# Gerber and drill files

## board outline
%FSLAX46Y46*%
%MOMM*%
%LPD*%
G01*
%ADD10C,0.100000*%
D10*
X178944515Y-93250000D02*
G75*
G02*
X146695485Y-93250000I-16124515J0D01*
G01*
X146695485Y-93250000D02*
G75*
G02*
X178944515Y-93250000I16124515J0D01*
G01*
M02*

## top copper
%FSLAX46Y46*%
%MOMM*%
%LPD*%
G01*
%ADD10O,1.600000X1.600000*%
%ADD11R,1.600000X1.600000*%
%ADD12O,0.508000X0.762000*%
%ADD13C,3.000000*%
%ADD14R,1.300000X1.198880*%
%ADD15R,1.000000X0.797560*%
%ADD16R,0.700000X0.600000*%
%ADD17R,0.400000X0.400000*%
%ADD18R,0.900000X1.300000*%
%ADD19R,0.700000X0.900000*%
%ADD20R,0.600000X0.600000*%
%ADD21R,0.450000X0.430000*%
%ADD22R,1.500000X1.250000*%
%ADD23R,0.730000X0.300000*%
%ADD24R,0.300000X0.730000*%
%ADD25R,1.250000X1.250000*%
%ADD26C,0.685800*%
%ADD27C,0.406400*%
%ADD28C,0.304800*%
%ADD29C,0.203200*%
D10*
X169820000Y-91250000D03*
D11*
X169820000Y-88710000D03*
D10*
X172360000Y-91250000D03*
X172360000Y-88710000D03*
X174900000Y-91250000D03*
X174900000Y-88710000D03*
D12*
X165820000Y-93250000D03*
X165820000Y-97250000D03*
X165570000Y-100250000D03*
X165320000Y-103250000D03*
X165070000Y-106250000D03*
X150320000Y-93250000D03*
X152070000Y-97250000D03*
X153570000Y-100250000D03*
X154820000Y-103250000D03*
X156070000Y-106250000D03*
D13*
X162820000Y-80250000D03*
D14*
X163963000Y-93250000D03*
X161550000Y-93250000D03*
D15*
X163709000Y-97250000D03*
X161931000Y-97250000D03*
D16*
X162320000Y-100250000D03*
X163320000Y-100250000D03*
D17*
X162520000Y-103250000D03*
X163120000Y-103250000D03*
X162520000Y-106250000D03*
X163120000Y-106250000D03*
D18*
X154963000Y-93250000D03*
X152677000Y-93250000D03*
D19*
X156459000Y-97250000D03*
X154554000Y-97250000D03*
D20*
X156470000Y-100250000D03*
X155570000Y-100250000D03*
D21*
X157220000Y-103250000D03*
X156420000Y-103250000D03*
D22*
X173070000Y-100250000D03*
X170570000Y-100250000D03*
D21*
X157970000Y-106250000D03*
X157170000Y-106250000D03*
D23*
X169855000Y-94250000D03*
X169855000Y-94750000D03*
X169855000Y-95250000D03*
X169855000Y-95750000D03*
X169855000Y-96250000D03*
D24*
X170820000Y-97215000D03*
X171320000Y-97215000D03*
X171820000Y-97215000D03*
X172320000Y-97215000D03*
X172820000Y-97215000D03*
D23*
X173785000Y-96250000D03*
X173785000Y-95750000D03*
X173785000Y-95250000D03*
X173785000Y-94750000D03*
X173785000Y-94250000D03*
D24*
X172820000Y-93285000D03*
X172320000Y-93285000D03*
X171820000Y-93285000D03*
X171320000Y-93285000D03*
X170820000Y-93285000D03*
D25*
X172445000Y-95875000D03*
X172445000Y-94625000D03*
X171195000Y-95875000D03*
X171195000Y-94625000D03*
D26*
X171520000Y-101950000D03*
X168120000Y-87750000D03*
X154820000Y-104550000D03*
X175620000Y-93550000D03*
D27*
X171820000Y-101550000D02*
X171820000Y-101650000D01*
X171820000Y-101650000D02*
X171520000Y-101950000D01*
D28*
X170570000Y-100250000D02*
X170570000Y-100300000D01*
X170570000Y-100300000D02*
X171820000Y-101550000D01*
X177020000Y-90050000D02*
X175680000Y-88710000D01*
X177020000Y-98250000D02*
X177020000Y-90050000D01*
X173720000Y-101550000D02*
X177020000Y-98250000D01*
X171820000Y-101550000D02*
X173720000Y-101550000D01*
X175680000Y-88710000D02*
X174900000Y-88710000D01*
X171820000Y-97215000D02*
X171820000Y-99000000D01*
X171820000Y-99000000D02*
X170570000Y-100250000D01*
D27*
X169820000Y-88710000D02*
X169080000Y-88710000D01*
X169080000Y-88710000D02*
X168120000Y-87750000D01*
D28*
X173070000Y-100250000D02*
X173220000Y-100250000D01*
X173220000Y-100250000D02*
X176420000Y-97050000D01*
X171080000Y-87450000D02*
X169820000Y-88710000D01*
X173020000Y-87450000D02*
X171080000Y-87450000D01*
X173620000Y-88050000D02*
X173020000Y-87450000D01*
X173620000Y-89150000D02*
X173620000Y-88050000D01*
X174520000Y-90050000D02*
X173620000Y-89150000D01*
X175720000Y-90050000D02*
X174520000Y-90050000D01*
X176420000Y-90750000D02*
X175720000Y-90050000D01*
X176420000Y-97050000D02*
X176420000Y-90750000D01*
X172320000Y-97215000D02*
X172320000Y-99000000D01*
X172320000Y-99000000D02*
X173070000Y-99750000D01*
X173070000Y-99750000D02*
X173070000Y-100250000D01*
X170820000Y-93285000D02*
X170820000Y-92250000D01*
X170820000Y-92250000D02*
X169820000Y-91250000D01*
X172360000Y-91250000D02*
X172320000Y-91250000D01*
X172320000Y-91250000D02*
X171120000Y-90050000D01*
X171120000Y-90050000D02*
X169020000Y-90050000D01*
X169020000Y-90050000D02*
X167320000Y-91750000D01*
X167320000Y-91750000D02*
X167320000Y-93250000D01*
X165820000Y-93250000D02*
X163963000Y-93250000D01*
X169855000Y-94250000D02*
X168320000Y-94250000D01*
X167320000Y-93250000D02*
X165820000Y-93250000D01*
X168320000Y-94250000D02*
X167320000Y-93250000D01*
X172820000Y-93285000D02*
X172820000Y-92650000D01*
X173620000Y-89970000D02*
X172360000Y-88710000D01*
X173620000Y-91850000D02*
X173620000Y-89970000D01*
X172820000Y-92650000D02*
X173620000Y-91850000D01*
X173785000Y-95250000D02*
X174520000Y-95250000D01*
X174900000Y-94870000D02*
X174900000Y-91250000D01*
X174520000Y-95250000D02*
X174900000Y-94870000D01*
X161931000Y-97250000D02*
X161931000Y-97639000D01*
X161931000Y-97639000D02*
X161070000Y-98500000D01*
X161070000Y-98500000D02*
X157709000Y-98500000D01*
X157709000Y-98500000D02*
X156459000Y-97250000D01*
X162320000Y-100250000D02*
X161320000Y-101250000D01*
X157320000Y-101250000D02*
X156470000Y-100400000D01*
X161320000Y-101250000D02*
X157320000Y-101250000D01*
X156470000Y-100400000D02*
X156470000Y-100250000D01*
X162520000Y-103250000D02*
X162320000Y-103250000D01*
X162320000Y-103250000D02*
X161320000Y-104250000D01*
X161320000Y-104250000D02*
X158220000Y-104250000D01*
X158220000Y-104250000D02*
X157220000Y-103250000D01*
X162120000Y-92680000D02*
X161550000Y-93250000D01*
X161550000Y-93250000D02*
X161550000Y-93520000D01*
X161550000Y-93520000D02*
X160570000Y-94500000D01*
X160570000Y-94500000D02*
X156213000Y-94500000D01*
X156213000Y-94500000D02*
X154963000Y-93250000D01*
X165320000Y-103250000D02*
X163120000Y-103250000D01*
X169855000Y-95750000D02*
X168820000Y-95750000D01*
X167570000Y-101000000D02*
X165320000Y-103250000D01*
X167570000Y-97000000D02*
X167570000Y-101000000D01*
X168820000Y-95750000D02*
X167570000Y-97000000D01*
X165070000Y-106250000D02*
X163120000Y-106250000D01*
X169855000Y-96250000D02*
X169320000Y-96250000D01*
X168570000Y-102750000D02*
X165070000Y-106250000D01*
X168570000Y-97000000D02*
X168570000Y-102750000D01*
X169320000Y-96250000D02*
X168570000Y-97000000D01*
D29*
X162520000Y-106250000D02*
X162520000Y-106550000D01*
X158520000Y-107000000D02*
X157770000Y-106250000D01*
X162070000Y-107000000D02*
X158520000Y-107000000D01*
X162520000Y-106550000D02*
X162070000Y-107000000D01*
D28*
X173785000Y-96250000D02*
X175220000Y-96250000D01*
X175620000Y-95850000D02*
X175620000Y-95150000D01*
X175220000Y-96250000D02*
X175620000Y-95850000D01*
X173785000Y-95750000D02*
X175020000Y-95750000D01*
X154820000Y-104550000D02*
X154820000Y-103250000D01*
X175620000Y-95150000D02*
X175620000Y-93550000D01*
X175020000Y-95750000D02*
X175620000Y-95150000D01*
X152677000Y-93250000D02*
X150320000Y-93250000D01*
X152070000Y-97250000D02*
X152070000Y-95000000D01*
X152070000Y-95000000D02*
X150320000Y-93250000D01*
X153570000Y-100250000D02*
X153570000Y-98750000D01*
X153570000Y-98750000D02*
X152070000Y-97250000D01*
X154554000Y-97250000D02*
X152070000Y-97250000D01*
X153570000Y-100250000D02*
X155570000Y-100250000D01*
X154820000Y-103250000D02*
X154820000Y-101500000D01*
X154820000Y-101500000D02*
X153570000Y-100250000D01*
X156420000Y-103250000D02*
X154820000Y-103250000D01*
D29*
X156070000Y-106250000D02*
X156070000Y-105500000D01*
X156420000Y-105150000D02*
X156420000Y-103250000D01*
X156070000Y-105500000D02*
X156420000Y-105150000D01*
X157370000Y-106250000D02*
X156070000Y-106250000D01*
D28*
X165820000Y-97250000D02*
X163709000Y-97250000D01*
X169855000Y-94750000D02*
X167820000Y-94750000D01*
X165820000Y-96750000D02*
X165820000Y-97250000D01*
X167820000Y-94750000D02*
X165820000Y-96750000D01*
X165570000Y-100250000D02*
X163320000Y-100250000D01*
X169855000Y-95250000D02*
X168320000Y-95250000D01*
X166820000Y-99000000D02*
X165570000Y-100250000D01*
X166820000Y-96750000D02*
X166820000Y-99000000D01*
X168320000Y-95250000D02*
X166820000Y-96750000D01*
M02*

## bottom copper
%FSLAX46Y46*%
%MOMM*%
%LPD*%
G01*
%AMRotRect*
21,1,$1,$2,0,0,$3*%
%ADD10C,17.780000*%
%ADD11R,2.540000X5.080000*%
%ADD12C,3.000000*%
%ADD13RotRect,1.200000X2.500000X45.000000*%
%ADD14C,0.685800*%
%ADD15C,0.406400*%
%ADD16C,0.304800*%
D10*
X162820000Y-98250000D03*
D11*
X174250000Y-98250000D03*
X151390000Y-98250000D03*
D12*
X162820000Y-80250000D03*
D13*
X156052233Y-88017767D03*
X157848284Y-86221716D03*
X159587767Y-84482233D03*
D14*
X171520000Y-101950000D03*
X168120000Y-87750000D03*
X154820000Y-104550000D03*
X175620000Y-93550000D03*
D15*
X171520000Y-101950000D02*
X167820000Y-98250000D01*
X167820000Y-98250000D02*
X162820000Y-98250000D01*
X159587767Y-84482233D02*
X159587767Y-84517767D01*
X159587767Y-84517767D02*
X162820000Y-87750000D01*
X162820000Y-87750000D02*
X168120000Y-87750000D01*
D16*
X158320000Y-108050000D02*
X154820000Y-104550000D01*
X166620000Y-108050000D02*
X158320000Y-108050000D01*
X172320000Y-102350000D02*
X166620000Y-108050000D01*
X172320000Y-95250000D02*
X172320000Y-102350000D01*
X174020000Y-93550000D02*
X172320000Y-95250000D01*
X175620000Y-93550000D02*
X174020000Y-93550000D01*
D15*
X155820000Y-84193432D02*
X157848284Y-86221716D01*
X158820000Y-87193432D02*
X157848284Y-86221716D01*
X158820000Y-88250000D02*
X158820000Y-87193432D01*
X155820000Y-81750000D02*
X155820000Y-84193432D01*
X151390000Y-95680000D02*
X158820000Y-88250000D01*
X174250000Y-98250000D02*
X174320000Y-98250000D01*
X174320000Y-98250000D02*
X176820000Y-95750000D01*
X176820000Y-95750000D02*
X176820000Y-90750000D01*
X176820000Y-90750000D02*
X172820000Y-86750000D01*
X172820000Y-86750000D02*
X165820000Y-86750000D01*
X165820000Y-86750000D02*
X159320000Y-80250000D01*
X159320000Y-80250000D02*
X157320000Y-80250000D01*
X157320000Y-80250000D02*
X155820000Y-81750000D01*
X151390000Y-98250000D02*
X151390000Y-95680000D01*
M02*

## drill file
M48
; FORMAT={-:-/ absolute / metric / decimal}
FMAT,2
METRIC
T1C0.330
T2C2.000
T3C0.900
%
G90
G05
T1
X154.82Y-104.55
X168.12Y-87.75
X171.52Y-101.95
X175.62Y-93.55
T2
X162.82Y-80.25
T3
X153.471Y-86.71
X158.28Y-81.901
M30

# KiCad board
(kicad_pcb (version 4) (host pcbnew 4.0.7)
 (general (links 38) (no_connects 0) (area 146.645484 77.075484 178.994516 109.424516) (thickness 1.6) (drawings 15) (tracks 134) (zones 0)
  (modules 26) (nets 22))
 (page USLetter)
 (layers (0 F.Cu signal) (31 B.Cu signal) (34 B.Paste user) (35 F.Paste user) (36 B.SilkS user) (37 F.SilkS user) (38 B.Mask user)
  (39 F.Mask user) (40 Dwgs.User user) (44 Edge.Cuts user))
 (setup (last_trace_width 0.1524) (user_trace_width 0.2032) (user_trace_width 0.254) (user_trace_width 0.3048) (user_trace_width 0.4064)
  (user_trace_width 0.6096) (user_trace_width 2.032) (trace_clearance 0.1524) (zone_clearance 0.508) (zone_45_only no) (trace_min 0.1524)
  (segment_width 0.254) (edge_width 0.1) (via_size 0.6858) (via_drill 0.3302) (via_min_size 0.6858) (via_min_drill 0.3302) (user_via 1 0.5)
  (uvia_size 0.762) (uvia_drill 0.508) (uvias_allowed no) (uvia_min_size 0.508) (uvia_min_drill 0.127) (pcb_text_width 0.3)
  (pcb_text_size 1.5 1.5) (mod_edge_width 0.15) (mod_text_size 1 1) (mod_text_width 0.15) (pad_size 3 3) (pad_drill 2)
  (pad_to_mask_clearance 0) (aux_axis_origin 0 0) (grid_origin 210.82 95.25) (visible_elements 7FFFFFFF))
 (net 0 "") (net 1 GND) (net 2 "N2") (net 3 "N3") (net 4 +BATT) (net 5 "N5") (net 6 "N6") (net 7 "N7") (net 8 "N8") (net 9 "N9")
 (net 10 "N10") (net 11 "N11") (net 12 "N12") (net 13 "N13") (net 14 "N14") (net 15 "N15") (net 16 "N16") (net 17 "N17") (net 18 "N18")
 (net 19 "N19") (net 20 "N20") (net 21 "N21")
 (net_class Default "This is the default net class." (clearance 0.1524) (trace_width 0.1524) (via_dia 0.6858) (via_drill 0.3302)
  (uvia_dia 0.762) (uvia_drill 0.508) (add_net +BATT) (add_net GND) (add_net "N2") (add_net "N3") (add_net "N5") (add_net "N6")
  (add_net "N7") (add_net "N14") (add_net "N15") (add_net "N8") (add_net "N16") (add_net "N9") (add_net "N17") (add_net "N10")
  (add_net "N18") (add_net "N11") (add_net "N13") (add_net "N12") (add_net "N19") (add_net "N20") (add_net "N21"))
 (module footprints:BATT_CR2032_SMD (layer B.Cu) (at 162.82 98.25 180)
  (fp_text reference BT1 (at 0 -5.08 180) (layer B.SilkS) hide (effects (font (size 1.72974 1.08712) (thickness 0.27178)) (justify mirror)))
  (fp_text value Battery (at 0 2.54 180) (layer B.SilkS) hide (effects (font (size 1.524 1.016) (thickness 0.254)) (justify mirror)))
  (pad 2 smd circle (at 0 0 180) (size 17.78 17.78) (layers B.Cu B.Paste B.Mask) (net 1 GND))
  (pad 1 smd rect (at -11.43 0 180) (size 2.54 5.08) (layers B.Cu B.Paste B.Mask) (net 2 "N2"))
  (pad 1 smd rect (at 11.43 0 180) (size 2.54 5.08) (layers B.Cu B.Paste B.Mask) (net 2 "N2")))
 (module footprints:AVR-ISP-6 (layer F.Cu) (at 169.82 91.25 90)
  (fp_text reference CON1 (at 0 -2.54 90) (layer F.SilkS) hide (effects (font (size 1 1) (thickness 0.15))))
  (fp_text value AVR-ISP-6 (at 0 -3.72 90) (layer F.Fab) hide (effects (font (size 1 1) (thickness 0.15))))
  (pad 1 smd oval (at 0 0 90) (size 1.6 1.6) (layers F.Cu F.Paste F.Mask) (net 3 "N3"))
  (pad 2 smd rect (at 2.54 0 90) (size 1.6 1.6) (layers F.Cu F.Paste F.Mask) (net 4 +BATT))
  (pad 3 smd oval (at 0 2.54 90) (size 1.6 1.6) (layers F.Cu F.Paste F.Mask) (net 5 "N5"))
  (pad 4 smd oval (at 2.54 2.54 90) (size 1.6 1.6) (layers F.Cu F.Paste F.Mask) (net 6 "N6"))
  (pad 5 smd oval (at 0 5.08 90) (size 1.6 1.6) (layers F.Cu F.Paste F.Mask) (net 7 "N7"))
  (pad 6 smd oval (at 2.54 5.08 90) (size 1.6 1.6) (layers F.Cu F.Paste F.Mask) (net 1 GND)))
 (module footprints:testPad (layer F.Cu) (at 165.82 93.25)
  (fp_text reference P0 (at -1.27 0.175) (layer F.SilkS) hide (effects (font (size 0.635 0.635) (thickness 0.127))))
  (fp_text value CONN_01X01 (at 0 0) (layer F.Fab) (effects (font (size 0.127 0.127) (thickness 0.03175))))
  (pad 1 smd oval (at 0 0) (size 0.508 0.762) (layers F.Cu F.Paste F.Mask) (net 5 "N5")))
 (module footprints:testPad (layer F.Cu) (at 165.82 97.25)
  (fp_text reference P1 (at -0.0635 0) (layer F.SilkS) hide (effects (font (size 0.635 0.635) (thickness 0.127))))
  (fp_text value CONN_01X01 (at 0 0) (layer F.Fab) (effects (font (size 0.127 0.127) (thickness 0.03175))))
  (pad 1 smd oval (at 0 0) (size 0.508 0.762) (layers F.Cu F.Paste F.Mask) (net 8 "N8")))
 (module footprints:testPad (layer F.Cu) (at 165.57 100.25)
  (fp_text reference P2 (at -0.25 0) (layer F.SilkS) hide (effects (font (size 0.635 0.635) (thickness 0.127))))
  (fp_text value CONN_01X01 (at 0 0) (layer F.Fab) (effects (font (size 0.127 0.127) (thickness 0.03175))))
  (pad 1 smd oval (at 0 0) (size 0.508 0.762) (layers F.Cu F.Paste F.Mask) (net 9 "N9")))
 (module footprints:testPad (layer F.Cu) (at 165.32 103.25)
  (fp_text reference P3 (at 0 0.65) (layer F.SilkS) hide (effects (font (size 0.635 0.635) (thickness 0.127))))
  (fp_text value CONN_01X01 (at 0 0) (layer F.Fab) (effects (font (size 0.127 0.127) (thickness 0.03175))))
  (pad 1 smd oval (at 0 0) (size 0.508 0.762) (layers F.Cu F.Paste F.Mask) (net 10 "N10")))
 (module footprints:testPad (layer F.Cu) (at 165.07 106.25)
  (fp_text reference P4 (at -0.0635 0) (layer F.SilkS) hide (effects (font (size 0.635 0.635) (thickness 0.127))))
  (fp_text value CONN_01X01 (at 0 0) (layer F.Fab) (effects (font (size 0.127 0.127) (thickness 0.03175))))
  (pad 1 smd oval (at 0 0) (size 0.508 0.762) (layers F.Cu F.Paste F.Mask) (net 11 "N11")))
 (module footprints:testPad (layer F.Cu) (at 150.32 93.25)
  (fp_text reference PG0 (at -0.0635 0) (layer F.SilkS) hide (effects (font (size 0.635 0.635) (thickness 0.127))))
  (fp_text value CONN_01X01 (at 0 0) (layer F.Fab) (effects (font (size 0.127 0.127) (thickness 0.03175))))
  (pad 1 smd oval (at 0 0) (size 0.508 0.762) (layers F.Cu F.Paste F.Mask) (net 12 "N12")))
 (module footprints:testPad (layer F.Cu) (at 152.07 97.25)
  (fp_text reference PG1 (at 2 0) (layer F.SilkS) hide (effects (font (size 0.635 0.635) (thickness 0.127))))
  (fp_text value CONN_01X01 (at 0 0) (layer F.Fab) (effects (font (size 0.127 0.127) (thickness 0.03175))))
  (pad 1 smd oval (at 0 0) (size 0.508 0.762) (layers F.Cu F.Paste F.Mask) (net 12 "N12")))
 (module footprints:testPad (layer F.Cu) (at 153.57 100.25)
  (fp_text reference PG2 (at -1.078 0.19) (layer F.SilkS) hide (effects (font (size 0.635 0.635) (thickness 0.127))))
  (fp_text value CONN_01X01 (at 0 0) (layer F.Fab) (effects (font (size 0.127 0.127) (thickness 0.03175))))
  (pad 1 smd oval (at 0 0) (size 0.508 0.762) (layers F.Cu F.Paste F.Mask) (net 12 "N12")))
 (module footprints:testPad (layer F.Cu) (at 154.82 103.25)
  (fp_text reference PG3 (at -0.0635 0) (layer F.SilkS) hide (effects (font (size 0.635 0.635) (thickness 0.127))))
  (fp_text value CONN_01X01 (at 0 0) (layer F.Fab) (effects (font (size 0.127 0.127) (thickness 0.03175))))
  (pad 1 smd oval (at 0 0) (size 0.508 0.762) (layers F.Cu F.Paste F.Mask) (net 12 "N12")))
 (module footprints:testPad (layer F.Cu) (at 156.07 106.25)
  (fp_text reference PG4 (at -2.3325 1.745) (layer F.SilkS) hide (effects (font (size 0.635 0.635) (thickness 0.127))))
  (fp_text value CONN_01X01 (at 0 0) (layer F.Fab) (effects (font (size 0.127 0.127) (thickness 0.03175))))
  (pad 1 smd oval (at 0 0) (size 0.508 0.762) (layers F.Cu F.Paste F.Mask) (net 12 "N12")))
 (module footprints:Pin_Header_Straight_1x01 (layer F.Cu) (at 162.82 80.25)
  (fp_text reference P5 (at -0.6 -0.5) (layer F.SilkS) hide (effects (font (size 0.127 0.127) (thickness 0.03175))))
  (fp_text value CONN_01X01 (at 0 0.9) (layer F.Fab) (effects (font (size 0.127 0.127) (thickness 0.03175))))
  (pad 1 thru_hole circle (at 0 0) (size 3 3) (drill 2) (layers *.Cu *.Mask) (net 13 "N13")))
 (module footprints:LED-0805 (layer F.Cu) (at 162.82 93.25)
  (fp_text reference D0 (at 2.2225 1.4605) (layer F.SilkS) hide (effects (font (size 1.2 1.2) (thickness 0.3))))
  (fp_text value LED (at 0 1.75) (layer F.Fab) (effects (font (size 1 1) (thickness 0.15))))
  (pad 2 smd rect (at 1.143 0 180) (size 1.3 1.19888) (layers F.Cu F.Paste F.Mask) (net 5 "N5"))
  (pad 1 smd rect (at -1.27 0 180) (size 1.3 1.19888) (layers F.Cu F.Paste F.Mask) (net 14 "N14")))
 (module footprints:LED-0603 (layer F.Cu) (at 162.82 97.25)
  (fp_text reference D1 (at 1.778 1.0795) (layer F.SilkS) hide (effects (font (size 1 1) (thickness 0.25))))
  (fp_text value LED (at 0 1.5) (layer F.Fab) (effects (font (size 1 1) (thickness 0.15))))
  (pad 2 smd rect (at 0.889 0 180) (size 1 0.79756) (layers F.Cu F.Paste F.Mask) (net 8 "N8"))
  (pad 1 smd rect (at -0.889 0 180) (size 1 0.79756) (layers F.Cu F.Paste F.Mask) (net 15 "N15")))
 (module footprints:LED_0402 (layer F.Cu) (at 162.82 100.25)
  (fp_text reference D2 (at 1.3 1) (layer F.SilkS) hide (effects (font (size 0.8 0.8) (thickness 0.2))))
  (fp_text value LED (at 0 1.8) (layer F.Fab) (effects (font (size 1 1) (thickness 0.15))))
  (pad 1 smd rect (at -0.5 0) (size 0.7 0.6) (layers F.Cu F.Paste F.Mask) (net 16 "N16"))
  (pad 2 smd rect (at 0.5 0) (size 0.7 0.6) (layers F.Cu F.Paste F.Mask) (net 9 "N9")))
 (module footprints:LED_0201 (layer F.Cu) (at 162.82 103.25)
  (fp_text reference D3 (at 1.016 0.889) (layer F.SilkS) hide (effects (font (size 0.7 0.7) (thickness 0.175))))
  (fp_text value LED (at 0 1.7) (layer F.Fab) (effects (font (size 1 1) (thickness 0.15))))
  (pad 1 smd rect (at -0.3 0) (size 0.4 0.4) (layers F.Cu F.Paste F.Mask) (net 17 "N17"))
  (pad 2 smd rect (at 0.3 0) (size 0.4 0.4) (layers F.Cu F.Paste F.Mask) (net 10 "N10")))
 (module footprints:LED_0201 (layer F.Cu) (at 162.82 106.25)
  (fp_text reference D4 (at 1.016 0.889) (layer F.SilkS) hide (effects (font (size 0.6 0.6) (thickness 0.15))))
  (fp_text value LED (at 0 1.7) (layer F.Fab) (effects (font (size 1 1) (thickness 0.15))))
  (pad 1 smd rect (at -0.3 0) (size 0.4 0.4) (layers F.Cu F.Paste F.Mask) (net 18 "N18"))
  (pad 2 smd rect (at 0.3 0) (size 0.4 0.4) (layers F.Cu F.Paste F.Mask) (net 11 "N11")))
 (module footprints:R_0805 (layer F.Cu) (at 153.82 93.25 180)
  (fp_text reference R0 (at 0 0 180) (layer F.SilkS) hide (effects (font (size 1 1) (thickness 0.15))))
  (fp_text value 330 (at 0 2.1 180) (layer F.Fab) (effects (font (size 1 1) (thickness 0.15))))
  (pad 1 smd rect (at -1.143 0 180) (size 0.9 1.3) (layers F.Cu F.Paste F.Mask) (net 14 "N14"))
  (pad 2 smd rect (at 1.143 0 180) (size 0.9 1.3) (layers F.Cu F.Paste F.Mask) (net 12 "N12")))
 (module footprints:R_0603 (layer F.Cu) (at 155.57 97.25 180)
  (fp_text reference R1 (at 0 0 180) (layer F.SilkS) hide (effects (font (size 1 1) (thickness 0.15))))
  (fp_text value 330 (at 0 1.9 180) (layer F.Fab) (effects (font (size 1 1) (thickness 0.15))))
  (pad 1 smd rect (at -0.889 0 180) (size 0.7 0.9) (layers F.Cu F.Paste F.Mask) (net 15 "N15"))
  (pad 2 smd rect (at 1.016 0 180) (size 0.7 0.9) (layers F.Cu F.Paste F.Mask) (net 12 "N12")))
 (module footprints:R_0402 (layer F.Cu) (at 156.07 100.25 180)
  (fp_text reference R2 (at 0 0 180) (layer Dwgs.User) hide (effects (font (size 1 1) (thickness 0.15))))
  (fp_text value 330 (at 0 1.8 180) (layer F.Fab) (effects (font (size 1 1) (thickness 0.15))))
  (pad 1 smd rect (at -0.4 0 180) (size 0.6 0.6) (layers F.Cu F.Paste F.Mask) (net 16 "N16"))
  (pad 2 smd rect (at 0.5 0 180) (size 0.6 0.6) (layers F.Cu F.Paste F.Mask) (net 12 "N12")))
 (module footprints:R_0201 (layer F.Cu) (at 156.82 103.25 180)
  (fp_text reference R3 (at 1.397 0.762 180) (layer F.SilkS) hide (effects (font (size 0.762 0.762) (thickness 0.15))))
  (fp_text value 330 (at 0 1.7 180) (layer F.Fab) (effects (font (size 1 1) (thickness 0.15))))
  (pad 1 smd rect (at -0.4 0 180) (size 0.45 0.43) (layers F.Cu F.Paste F.Mask) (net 17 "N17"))
  (pad 2 smd rect (at 0.4 0 180) (size 0.45 0.43) (layers F.Cu F.Paste F.Mask) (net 12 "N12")))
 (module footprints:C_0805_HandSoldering (layer F.Cu) (at 171.82 100.25 180)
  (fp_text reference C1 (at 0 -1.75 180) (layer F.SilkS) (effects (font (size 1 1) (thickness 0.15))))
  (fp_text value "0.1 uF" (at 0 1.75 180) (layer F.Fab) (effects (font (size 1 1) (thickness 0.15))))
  (pad 1 smd rect (at -1.25 0 180) (size 1.5 1.25) (layers F.Cu F.Paste F.Mask) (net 4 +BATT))
  (pad 2 smd rect (at 1.25 0 180) (size 1.5 1.25) (layers F.Cu F.Paste F.Mask) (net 1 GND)))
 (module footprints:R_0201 (layer F.Cu) (at 157.57 106.25 180)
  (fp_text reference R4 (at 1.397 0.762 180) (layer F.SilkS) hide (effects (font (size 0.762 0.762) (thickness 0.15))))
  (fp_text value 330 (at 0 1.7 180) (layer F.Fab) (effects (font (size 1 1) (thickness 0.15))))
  (pad 1 smd rect (at -0.4 0 180) (size 0.45 0.43) (layers F.Cu F.Paste F.Mask) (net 18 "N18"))
  (pad 2 smd rect (at 0.4 0 180) (size 0.45 0.43) (layers F.Cu F.Paste F.Mask) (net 12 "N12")))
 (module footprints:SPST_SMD (layer B.Cu) (at 157.82 86.25 45)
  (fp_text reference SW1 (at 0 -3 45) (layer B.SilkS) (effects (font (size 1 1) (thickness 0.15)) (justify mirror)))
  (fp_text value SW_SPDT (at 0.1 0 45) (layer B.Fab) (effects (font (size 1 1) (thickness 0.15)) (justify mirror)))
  (pad "" np_thru_hole circle (at 3.4 -2.75 45) (size 0.9 0.9) (drill 0.9) (layers *.Cu *.Mask))
  (pad 1 smd rect (at -2.5 0 45) (size 1.2 2.5) (layers B.Cu B.Paste B.Mask) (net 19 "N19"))
  (pad 2 smd rect (at 0.04 0 45) (size 1.2 2.5) (layers B.Cu B.Paste B.Mask) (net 2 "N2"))
  (pad 3 smd rect (at 2.5 0 45) (size 1.2 2.5) (layers B.Cu B.Paste B.Mask) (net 4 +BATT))
  (pad "" np_thru_hole circle (at -3.4 -2.75 45) (size 0.9 0.9) (drill 0.9) (layers *.Cu *.Mask)))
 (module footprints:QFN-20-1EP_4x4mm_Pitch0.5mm (layer F.Cu) (at 171.82 95.25)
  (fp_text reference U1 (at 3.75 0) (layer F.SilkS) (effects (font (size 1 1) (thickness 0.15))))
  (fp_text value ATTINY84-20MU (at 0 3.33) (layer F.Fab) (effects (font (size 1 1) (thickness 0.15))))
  (pad 1 smd rect (at -1.965 -1) (size 0.73 0.3) (layers F.Cu F.Paste F.Mask) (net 5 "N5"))
  (pad 2 smd rect (at -1.965 -0.5) (size 0.73 0.3) (layers F.Cu F.Paste F.Mask) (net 8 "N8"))
  (pad 3 smd rect (at -1.965 0) (size 0.73 0.3) (layers F.Cu F.Paste F.Mask) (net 9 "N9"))
  (pad 4 smd rect (at -1.965 0.5) (size 0.73 0.3) (layers F.Cu F.Paste F.Mask) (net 10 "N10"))
  (pad 5 smd rect (at -1.965 1) (size 0.73 0.3) (layers F.Cu F.Paste F.Mask) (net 11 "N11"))
  (pad 6 smd rect (at -1 1.965 90) (size 0.73 0.3) (layers F.Cu F.Paste F.Mask))
  (pad 7 smd rect (at -0.5 1.965 90) (size 0.73 0.3) (layers F.Cu F.Paste F.Mask))
  (pad 8 smd rect (at 0 1.965 90) (size 0.73 0.3) (layers F.Cu F.Paste F.Mask) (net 1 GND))
  (pad 9 smd rect (at 0.5 1.965 90) (size 0.73 0.3) (layers F.Cu F.Paste F.Mask) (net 4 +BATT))
  (pad 10 smd rect (at 1 1.965 90) (size 0.73 0.3) (layers F.Cu F.Paste F.Mask))
  (pad 11 smd rect (at 1.965 1) (size 0.73 0.3) (layers F.Cu F.Paste F.Mask) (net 12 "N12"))
  (pad 12 smd rect (at 1.965 0.5) (size 0.73 0.3) (layers F.Cu F.Paste F.Mask) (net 12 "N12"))
  (pad 13 smd rect (at 1.965 0) (size 0.73 0.3) (layers F.Cu F.Paste F.Mask) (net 7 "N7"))
  (pad 14 smd rect (at 1.965 -0.5) (size 0.73 0.3) (layers F.Cu F.Paste F.Mask) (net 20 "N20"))
  (pad 15 smd rect (at 1.965 -1) (size 0.73 0.3) (layers F.Cu F.Paste F.Mask) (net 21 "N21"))
  (pad 16 smd rect (at 1 -1.965 90) (size 0.73 0.3) (layers F.Cu F.Paste F.Mask) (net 6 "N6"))
  (pad 17 smd rect (at 0.5 -1.965 90) (size 0.73 0.3) (layers F.Cu F.Paste F.Mask))
  (pad 18 smd rect (at 0 -1.965 90) (size 0.73 0.3) (layers F.Cu F.Paste F.Mask))
  (pad 19 smd rect (at -0.5 -1.965 90) (size 0.73 0.3) (layers F.Cu F.Paste F.Mask))
  (pad 20 smd rect (at -1 -1.965 90) (size 0.73 0.3) (layers F.Cu F.Paste F.Mask) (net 3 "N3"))
  (pad 21 smd rect (at 0.625 0.625) (size 1.25 1.25) (layers F.Cu F.Paste F.Mask) (solder_paste_margin_ratio -0.2))
  (pad 21 smd rect (at 0.625 -0.625) (size 1.25 1.25) (layers F.Cu F.Paste F.Mask) (solder_paste_margin_ratio -0.2))
  (pad 21 smd rect (at -0.625 0.625) (size 1.25 1.25) (layers F.Cu F.Paste F.Mask) (solder_paste_margin_ratio -0.2))
  (pad 21 smd rect (at -0.625 -0.625) (size 1.25 1.25) (layers F.Cu F.Paste F.Mask) (solder_paste_margin_ratio -0.2)))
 (gr_circle (center 162.82 93.25) (end 148.82 85.25) (layer Edge.Cuts) (width 0.1))
 (segment (start 171.82 101.55) (end 171.82 101.65) (width 0.4064) (layer F.Cu) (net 1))
 (segment (start 171.52 101.95) (end 167.82 98.25) (width 0.4064) (layer B.Cu) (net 1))
 (via (at 171.52 101.95) (size 0.6858) (drill 0.3302) (layers F.Cu B.Cu) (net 1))
 (segment (start 171.82 101.65) (end 171.52 101.95) (width 0.4064) (layer F.Cu) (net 1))
 (segment (start 167.82 98.25) (end 162.82 98.25) (width 0.4064) (layer B.Cu) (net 1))
 (segment (start 170.57 100.25) (end 170.57 100.3) (width 0.3048) (layer F.Cu) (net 1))
 (segment (start 170.57 100.3) (end 171.82 101.55) (width 0.3048) (layer F.Cu) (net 1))
 (segment (start 177.02 90.05) (end 175.68 88.71) (width 0.3048) (layer F.Cu) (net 1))
 (segment (start 177.02 98.25) (end 177.02 90.05) (width 0.3048) (layer F.Cu) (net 1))
 (segment (start 173.72 101.55) (end 177.02 98.25) (width 0.3048) (layer F.Cu) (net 1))
 (segment (start 171.82 101.55) (end 173.72 101.55) (width 0.3048) (layer F.Cu) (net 1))
 (segment (start 175.68 88.71) (end 174.9 88.71) (width 0.3048) (layer F.Cu) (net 1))
 (segment (start 171.82 97.215) (end 171.82 99) (width 0.3048) (layer F.Cu) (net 1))
 (segment (start 171.82 99) (end 170.57 100.25) (width 0.3048) (layer F.Cu) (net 1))
 (segment (start 169.82 88.71) (end 169.08 88.71) (width 0.4064) (layer F.Cu) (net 4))
 (segment (start 169.08 88.71) (end 168.12 87.75) (width 0.4064) (layer F.Cu) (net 4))
 (segment (start 173.07 100.25) (end 173.22 100.25) (width 0.3048) (layer F.Cu) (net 4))
 (segment (start 173.22 100.25) (end 176.42 97.05) (width 0.3048) (layer F.Cu) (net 4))
 (segment (start 171.08 87.45) (end 169.82 88.71) (width 0.3048) (layer F.Cu) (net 4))
 (segment (start 173.02 87.45) (end 171.08 87.45) (width 0.3048) (layer F.Cu) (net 4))
 (segment (start 173.62 88.05) (end 173.02 87.45) (width 0.3048) (layer F.Cu) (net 4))
 (segment (start 173.62 89.15) (end 173.62 88.05) (width 0.3048) (layer F.Cu) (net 4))
 (segment (start 174.52 90.05) (end 173.62 89.15) (width 0.3048) (layer F.Cu) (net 4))
 (segment (start 175.72 90.05) (end 174.52 90.05) (width 0.3048) (layer F.Cu) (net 4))
 (segment (start 176.42 90.75) (end 175.72 90.05) (width 0.3048) (layer F.Cu) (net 4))
 (segment (start 176.42 97.05) (end 176.42 90.75) (width 0.3048) (layer F.Cu) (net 4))
 (segment (start 172.32 97.215) (end 172.32 99) (width 0.3048) (layer F.Cu) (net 4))
 (segment (start 172.32 99) (end 173.07 99.75) (width 0.3048) (layer F.Cu) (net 4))
 (segment (start 173.07 99.75) (end 173.07 100.25) (width 0.3048) (layer F.Cu) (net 4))
 (via (at 168.12 87.75) (size 0.6858) (drill 0.3302) (layers F.Cu B.Cu) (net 4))
 (segment (start 159.587767 84.482233) (end 159.587767 84.517767) (width 0.4064) (layer B.Cu) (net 4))
 (segment (start 159.587767 84.517767) (end 162.82 87.75) (width 0.4064) (layer B.Cu) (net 4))
 (segment (start 162.82 87.75) (end 168.12 87.75) (width 0.4064) (layer B.Cu) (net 4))
 (segment (start 170.82 93.285) (end 170.82 92.25) (width 0.3048) (layer F.Cu) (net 3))
 (segment (start 170.82 92.25) (end 169.82 91.25) (width 0.3048) (layer F.Cu) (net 3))
 (segment (start 172.36 91.25) (end 172.32 91.25) (width 0.3048) (layer F.Cu) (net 5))
 (segment (start 172.32 91.25) (end 171.12 90.05) (width 0.3048) (layer F.Cu) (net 5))
 (segment (start 171.12 90.05) (end 169.02 90.05) (width 0.3048) (layer F.Cu) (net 5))
 (segment (start 169.02 90.05) (end 167.32 91.75) (width 0.3048) (layer F.Cu) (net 5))
 (segment (start 167.32 91.75) (end 167.32 93.25) (width 0.3048) (layer F.Cu) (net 5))
 (segment (start 165.82 93.25) (end 163.963 93.25) (width 0.3048) (layer F.Cu) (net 5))
 (segment (start 169.855 94.25) (end 168.32 94.25) (width 0.3048) (layer F.Cu) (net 5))
 (segment (start 167.32 93.25) (end 165.82 93.25) (width 0.3048) (layer F.Cu) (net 5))
 (segment (start 168.32 94.25) (end 167.32 93.25) (width 0.3048) (layer F.Cu) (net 5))
 (segment (start 172.82 93.285) (end 172.82 92.65) (width 0.3048) (layer F.Cu) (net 6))
 (segment (start 173.62 89.97) (end 172.36 88.71) (width 0.3048) (layer F.Cu) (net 6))
 (segment (start 173.62 91.85) (end 173.62 89.97) (width 0.3048) (layer F.Cu) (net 6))
 (segment (start 172.82 92.65) (end 173.62 91.85) (width 0.3048) (layer F.Cu) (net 6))
 (segment (start 173.785 95.25) (end 174.52 95.25) (width 0.3048) (layer F.Cu) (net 7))
 (segment (start 174.9 94.87) (end 174.9 91.25) (width 0.3048) (layer F.Cu) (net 7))
 (segment (start 174.52 95.25) (end 174.9 94.87) (width 0.3048) (layer F.Cu) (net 7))
 (segment (start 161.931 97.25) (end 161.931 97.639) (width 0.3048) (layer F.Cu) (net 15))
 (segment (start 161.931 97.639) (end 161.07 98.5) (width 0.3048) (layer F.Cu) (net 15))
 (segment (start 161.07 98.5) (end 157.709 98.5) (width 0.3048) (layer F.Cu) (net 15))
 (segment (start 157.709 98.5) (end 156.459 97.25) (width 0.3048) (layer F.Cu) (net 15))
 (segment (start 162.32 100.25) (end 161.32 101.25) (width 0.3048) (layer F.Cu) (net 16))
 (segment (start 157.32 101.25) (end 156.47 100.4) (width 0.3048) (layer F.Cu) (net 16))
 (segment (start 161.32 101.25) (end 157.32 101.25) (width 0.3048) (layer F.Cu) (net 16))
 (segment (start 156.47 100.4) (end 156.47 100.25) (width 0.3048) (layer F.Cu) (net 16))
 (segment (start 162.52 103.25) (end 162.32 103.25) (width 0.3048) (layer F.Cu) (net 17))
 (segment (start 162.32 103.25) (end 161.32 104.25) (width 0.3048) (layer F.Cu) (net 17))
 (segment (start 161.32 104.25) (end 158.22 104.25) (width 0.3048) (layer F.Cu) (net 17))
 (segment (start 158.22 104.25) (end 157.22 103.25) (width 0.3048) (layer F.Cu) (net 17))
 (segment (start 162.12 92.68) (end 161.55 93.25) (width 0.3048) (layer F.Cu) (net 14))
 (segment (start 161.55 93.25) (end 161.55 93.52) (width 0.3048) (layer F.Cu) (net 14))
 (segment (start 161.55 93.52) (end 160.57 94.5) (width 0.3048) (layer F.Cu) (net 14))
 (segment (start 160.57 94.5) (end 156.213 94.5) (width 0.3048) (layer F.Cu) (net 14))
 (segment (start 156.213 94.5) (end 154.963 93.25) (width 0.3048) (layer F.Cu) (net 14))
 (segment (start 165.32 103.25) (end 163.12 103.25) (width 0.3048) (layer F.Cu) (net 10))
 (segment (start 169.855 95.75) (end 168.82 95.75) (width 0.3048) (layer F.Cu) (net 10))
 (segment (start 167.57 101) (end 165.32 103.25) (width 0.3048) (layer F.Cu) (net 10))
 (segment (start 167.57 97) (end 167.57 101) (width 0.3048) (layer F.Cu) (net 10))
 (segment (start 168.82 95.75) (end 167.57 97) (width 0.3048) (layer F.Cu) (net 10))
 (segment (start 165.07 106.25) (end 163.12 106.25) (width 0.3048) (layer F.Cu) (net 11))
 (segment (start 169.855 96.25) (end 169.32 96.25) (width 0.3048) (layer F.Cu) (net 11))
 (segment (start 168.57 102.75) (end 165.07 106.25) (width 0.3048) (layer F.Cu) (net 11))
 (segment (start 168.57 97) (end 168.57 102.75) (width 0.3048) (layer F.Cu) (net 11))
 (segment (start 169.32 96.25) (end 168.57 97) (width 0.3048) (layer F.Cu) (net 11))
 (segment (start 162.52 106.25) (end 162.52 106.55) (width 0.2032) (layer F.Cu) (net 18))
 (segment (start 158.52 107) (end 157.77 106.25) (width 0.2032) (layer F.Cu) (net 18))
 (segment (start 162.07 107) (end 158.52 107) (width 0.2032) (layer F.Cu) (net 18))
 (segment (start 162.52 106.55) (end 162.07 107) (width 0.2032) (layer F.Cu) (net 18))
 (segment (start 173.785 96.25) (end 175.22 96.25) (width 0.3048) (layer F.Cu) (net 12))
 (segment (start 175.62 95.85) (end 175.62 95.15) (width 0.3048) (layer F.Cu) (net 12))
 (segment (start 175.22 96.25) (end 175.62 95.85) (width 0.3048) (layer F.Cu) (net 12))
 (segment (start 173.785 95.75) (end 175.02 95.75) (width 0.3048) (layer F.Cu) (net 12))
 (segment (start 154.82 104.55) (end 154.82 103.25) (width 0.3048) (layer F.Cu) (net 12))
 (via (at 154.82 104.55) (size 0.6858) (drill 0.3302) (layers F.Cu B.Cu) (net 12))
 (segment (start 158.32 108.05) (end 154.82 104.55) (width 0.3048) (layer B.Cu) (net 12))
 (segment (start 166.62 108.05) (end 158.32 108.05) (width 0.3048) (layer B.Cu) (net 12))
 (segment (start 172.32 102.35) (end 166.62 108.05) (width 0.3048) (layer B.Cu) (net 12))
 (segment (start 172.32 95.25) (end 172.32 102.35) (width 0.3048) (layer B.Cu) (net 12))
 (segment (start 174.02 93.55) (end 172.32 95.25) (width 0.3048) (layer B.Cu) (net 12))
 (segment (start 175.62 93.55) (end 174.02 93.55) (width 0.3048) (layer B.Cu) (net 12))
 (via (at 175.62 93.55) (size 0.6858) (drill 0.3302) (layers F.Cu B.Cu) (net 12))
 (segment (start 175.62 95.15) (end 175.62 93.55) (width 0.3048) (layer F.Cu) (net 12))
 (segment (start 175.02 95.75) (end 175.62 95.15) (width 0.3048) (layer F.Cu) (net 12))
 (segment (start 152.677 93.25) (end 150.32 93.25) (width 0.3048) (layer F.Cu) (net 12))
 (segment (start 152.07 97.25) (end 152.07 95) (width 0.3048) (layer F.Cu) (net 12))
 (segment (start 152.07 95) (end 150.32 93.25) (width 0.3048) (layer F.Cu) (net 12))
 (segment (start 153.57 100.25) (end 153.57 98.75) (width 0.3048) (layer F.Cu) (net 12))
 (segment (start 153.57 98.75) (end 152.07 97.25) (width 0.3048) (layer F.Cu) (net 12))
 (segment (start 154.554 97.25) (end 152.07 97.25) (width 0.3048) (layer F.Cu) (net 12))
 (segment (start 153.57 100.25) (end 155.57 100.25) (width 0.3048) (layer F.Cu) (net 12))
 (segment (start 154.82 103.25) (end 154.82 101.5) (width 0.3048) (layer F.Cu) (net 12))
 (segment (start 154.82 101.5) (end 153.57 100.25) (width 0.3048) (layer F.Cu) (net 12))
 (segment (start 156.42 103.25) (end 154.82 103.25) (width 0.3048) (layer F.Cu) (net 12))
 (segment (start 156.07 106.25) (end 156.07 105.5) (width 0.2032) (layer F.Cu) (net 12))
 (segment (start 156.42 105.15) (end 156.42 103.25) (width 0.2032) (layer F.Cu) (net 12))
 (segment (start 156.07 105.5) (end 156.42 105.15) (width 0.2032) (layer F.Cu) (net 12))
 (segment (start 157.37 106.25) (end 156.07 106.25) (width 0.2032) (layer F.Cu) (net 12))
 (segment (start 165.82 97.25) (end 163.709 97.25) (width 0.3048) (layer F.Cu) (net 8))
 (segment (start 169.855 94.75) (end 167.82 94.75) (width 0.3048) (layer F.Cu) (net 8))
 (segment (start 165.82 96.75) (end 165.82 97.25) (width 0.3048) (layer F.Cu) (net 8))
 (segment (start 167.82 94.75) (end 165.82 96.75) (width 0.3048) (layer F.Cu) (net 8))
 (segment (start 165.57 100.25) (end 163.32 100.25) (width 0.3048) (layer F.Cu) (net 9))
 (segment (start 169.855 95.25) (end 168.32 95.25) (width 0.3048) (layer F.Cu) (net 9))
 (segment (start 166.82 99) (end 165.57 100.25) (width 0.3048) (layer F.Cu) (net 9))
 (segment (start 166.82 96.75) (end 166.82 99) (width 0.3048) (layer F.Cu) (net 9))
 (segment (start 168.32 95.25) (end 166.82 96.75) (width 0.3048) (layer F.Cu) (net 9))
 (segment (start 155.82 84.193432) (end 157.848284 86.221716) (width 0.4064) (layer B.Cu) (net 2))
 (segment (start 158.82 87.193432) (end 157.848284 86.221716) (width 0.4064) (layer B.Cu) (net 2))
 (segment (start 158.82 88.25) (end 158.82 87.193432) (width 0.4064) (layer B.Cu) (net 2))
 (segment (start 155.82 81.75) (end 155.82 84.193432) (width 0.4064) (layer B.Cu) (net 2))
 (segment (start 151.39 95.68) (end 158.82 88.25) (width 0.4064) (layer B.Cu) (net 2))
 (segment (start 174.25 98.25) (end 174.32 98.25) (width 0.4064) (layer B.Cu) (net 2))
 (segment (start 174.32 98.25) (end 176.82 95.75) (width 0.4064) (layer B.Cu) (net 2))
 (segment (start 176.82 95.75) (end 176.82 90.75) (width 0.4064) (layer B.Cu) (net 2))
 (segment (start 176.82 90.75) (end 172.82 86.75) (width 0.4064) (layer B.Cu) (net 2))
 (segment (start 172.82 86.75) (end 165.82 86.75) (width 0.4064) (layer B.Cu) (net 2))
 (segment (start 165.82 86.75) (end 159.32 80.25) (width 0.4064) (layer B.Cu) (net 2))
 (segment (start 159.32 80.25) (end 157.32 80.25) (width 0.4064) (layer B.Cu) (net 2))
 (segment (start 157.32 80.25) (end 155.82 81.75) (width 0.4064) (layer B.Cu) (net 2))
 (segment (start 151.39 98.25) (end 151.39 95.68) (width 0.4064) (layer B.Cu) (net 2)))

